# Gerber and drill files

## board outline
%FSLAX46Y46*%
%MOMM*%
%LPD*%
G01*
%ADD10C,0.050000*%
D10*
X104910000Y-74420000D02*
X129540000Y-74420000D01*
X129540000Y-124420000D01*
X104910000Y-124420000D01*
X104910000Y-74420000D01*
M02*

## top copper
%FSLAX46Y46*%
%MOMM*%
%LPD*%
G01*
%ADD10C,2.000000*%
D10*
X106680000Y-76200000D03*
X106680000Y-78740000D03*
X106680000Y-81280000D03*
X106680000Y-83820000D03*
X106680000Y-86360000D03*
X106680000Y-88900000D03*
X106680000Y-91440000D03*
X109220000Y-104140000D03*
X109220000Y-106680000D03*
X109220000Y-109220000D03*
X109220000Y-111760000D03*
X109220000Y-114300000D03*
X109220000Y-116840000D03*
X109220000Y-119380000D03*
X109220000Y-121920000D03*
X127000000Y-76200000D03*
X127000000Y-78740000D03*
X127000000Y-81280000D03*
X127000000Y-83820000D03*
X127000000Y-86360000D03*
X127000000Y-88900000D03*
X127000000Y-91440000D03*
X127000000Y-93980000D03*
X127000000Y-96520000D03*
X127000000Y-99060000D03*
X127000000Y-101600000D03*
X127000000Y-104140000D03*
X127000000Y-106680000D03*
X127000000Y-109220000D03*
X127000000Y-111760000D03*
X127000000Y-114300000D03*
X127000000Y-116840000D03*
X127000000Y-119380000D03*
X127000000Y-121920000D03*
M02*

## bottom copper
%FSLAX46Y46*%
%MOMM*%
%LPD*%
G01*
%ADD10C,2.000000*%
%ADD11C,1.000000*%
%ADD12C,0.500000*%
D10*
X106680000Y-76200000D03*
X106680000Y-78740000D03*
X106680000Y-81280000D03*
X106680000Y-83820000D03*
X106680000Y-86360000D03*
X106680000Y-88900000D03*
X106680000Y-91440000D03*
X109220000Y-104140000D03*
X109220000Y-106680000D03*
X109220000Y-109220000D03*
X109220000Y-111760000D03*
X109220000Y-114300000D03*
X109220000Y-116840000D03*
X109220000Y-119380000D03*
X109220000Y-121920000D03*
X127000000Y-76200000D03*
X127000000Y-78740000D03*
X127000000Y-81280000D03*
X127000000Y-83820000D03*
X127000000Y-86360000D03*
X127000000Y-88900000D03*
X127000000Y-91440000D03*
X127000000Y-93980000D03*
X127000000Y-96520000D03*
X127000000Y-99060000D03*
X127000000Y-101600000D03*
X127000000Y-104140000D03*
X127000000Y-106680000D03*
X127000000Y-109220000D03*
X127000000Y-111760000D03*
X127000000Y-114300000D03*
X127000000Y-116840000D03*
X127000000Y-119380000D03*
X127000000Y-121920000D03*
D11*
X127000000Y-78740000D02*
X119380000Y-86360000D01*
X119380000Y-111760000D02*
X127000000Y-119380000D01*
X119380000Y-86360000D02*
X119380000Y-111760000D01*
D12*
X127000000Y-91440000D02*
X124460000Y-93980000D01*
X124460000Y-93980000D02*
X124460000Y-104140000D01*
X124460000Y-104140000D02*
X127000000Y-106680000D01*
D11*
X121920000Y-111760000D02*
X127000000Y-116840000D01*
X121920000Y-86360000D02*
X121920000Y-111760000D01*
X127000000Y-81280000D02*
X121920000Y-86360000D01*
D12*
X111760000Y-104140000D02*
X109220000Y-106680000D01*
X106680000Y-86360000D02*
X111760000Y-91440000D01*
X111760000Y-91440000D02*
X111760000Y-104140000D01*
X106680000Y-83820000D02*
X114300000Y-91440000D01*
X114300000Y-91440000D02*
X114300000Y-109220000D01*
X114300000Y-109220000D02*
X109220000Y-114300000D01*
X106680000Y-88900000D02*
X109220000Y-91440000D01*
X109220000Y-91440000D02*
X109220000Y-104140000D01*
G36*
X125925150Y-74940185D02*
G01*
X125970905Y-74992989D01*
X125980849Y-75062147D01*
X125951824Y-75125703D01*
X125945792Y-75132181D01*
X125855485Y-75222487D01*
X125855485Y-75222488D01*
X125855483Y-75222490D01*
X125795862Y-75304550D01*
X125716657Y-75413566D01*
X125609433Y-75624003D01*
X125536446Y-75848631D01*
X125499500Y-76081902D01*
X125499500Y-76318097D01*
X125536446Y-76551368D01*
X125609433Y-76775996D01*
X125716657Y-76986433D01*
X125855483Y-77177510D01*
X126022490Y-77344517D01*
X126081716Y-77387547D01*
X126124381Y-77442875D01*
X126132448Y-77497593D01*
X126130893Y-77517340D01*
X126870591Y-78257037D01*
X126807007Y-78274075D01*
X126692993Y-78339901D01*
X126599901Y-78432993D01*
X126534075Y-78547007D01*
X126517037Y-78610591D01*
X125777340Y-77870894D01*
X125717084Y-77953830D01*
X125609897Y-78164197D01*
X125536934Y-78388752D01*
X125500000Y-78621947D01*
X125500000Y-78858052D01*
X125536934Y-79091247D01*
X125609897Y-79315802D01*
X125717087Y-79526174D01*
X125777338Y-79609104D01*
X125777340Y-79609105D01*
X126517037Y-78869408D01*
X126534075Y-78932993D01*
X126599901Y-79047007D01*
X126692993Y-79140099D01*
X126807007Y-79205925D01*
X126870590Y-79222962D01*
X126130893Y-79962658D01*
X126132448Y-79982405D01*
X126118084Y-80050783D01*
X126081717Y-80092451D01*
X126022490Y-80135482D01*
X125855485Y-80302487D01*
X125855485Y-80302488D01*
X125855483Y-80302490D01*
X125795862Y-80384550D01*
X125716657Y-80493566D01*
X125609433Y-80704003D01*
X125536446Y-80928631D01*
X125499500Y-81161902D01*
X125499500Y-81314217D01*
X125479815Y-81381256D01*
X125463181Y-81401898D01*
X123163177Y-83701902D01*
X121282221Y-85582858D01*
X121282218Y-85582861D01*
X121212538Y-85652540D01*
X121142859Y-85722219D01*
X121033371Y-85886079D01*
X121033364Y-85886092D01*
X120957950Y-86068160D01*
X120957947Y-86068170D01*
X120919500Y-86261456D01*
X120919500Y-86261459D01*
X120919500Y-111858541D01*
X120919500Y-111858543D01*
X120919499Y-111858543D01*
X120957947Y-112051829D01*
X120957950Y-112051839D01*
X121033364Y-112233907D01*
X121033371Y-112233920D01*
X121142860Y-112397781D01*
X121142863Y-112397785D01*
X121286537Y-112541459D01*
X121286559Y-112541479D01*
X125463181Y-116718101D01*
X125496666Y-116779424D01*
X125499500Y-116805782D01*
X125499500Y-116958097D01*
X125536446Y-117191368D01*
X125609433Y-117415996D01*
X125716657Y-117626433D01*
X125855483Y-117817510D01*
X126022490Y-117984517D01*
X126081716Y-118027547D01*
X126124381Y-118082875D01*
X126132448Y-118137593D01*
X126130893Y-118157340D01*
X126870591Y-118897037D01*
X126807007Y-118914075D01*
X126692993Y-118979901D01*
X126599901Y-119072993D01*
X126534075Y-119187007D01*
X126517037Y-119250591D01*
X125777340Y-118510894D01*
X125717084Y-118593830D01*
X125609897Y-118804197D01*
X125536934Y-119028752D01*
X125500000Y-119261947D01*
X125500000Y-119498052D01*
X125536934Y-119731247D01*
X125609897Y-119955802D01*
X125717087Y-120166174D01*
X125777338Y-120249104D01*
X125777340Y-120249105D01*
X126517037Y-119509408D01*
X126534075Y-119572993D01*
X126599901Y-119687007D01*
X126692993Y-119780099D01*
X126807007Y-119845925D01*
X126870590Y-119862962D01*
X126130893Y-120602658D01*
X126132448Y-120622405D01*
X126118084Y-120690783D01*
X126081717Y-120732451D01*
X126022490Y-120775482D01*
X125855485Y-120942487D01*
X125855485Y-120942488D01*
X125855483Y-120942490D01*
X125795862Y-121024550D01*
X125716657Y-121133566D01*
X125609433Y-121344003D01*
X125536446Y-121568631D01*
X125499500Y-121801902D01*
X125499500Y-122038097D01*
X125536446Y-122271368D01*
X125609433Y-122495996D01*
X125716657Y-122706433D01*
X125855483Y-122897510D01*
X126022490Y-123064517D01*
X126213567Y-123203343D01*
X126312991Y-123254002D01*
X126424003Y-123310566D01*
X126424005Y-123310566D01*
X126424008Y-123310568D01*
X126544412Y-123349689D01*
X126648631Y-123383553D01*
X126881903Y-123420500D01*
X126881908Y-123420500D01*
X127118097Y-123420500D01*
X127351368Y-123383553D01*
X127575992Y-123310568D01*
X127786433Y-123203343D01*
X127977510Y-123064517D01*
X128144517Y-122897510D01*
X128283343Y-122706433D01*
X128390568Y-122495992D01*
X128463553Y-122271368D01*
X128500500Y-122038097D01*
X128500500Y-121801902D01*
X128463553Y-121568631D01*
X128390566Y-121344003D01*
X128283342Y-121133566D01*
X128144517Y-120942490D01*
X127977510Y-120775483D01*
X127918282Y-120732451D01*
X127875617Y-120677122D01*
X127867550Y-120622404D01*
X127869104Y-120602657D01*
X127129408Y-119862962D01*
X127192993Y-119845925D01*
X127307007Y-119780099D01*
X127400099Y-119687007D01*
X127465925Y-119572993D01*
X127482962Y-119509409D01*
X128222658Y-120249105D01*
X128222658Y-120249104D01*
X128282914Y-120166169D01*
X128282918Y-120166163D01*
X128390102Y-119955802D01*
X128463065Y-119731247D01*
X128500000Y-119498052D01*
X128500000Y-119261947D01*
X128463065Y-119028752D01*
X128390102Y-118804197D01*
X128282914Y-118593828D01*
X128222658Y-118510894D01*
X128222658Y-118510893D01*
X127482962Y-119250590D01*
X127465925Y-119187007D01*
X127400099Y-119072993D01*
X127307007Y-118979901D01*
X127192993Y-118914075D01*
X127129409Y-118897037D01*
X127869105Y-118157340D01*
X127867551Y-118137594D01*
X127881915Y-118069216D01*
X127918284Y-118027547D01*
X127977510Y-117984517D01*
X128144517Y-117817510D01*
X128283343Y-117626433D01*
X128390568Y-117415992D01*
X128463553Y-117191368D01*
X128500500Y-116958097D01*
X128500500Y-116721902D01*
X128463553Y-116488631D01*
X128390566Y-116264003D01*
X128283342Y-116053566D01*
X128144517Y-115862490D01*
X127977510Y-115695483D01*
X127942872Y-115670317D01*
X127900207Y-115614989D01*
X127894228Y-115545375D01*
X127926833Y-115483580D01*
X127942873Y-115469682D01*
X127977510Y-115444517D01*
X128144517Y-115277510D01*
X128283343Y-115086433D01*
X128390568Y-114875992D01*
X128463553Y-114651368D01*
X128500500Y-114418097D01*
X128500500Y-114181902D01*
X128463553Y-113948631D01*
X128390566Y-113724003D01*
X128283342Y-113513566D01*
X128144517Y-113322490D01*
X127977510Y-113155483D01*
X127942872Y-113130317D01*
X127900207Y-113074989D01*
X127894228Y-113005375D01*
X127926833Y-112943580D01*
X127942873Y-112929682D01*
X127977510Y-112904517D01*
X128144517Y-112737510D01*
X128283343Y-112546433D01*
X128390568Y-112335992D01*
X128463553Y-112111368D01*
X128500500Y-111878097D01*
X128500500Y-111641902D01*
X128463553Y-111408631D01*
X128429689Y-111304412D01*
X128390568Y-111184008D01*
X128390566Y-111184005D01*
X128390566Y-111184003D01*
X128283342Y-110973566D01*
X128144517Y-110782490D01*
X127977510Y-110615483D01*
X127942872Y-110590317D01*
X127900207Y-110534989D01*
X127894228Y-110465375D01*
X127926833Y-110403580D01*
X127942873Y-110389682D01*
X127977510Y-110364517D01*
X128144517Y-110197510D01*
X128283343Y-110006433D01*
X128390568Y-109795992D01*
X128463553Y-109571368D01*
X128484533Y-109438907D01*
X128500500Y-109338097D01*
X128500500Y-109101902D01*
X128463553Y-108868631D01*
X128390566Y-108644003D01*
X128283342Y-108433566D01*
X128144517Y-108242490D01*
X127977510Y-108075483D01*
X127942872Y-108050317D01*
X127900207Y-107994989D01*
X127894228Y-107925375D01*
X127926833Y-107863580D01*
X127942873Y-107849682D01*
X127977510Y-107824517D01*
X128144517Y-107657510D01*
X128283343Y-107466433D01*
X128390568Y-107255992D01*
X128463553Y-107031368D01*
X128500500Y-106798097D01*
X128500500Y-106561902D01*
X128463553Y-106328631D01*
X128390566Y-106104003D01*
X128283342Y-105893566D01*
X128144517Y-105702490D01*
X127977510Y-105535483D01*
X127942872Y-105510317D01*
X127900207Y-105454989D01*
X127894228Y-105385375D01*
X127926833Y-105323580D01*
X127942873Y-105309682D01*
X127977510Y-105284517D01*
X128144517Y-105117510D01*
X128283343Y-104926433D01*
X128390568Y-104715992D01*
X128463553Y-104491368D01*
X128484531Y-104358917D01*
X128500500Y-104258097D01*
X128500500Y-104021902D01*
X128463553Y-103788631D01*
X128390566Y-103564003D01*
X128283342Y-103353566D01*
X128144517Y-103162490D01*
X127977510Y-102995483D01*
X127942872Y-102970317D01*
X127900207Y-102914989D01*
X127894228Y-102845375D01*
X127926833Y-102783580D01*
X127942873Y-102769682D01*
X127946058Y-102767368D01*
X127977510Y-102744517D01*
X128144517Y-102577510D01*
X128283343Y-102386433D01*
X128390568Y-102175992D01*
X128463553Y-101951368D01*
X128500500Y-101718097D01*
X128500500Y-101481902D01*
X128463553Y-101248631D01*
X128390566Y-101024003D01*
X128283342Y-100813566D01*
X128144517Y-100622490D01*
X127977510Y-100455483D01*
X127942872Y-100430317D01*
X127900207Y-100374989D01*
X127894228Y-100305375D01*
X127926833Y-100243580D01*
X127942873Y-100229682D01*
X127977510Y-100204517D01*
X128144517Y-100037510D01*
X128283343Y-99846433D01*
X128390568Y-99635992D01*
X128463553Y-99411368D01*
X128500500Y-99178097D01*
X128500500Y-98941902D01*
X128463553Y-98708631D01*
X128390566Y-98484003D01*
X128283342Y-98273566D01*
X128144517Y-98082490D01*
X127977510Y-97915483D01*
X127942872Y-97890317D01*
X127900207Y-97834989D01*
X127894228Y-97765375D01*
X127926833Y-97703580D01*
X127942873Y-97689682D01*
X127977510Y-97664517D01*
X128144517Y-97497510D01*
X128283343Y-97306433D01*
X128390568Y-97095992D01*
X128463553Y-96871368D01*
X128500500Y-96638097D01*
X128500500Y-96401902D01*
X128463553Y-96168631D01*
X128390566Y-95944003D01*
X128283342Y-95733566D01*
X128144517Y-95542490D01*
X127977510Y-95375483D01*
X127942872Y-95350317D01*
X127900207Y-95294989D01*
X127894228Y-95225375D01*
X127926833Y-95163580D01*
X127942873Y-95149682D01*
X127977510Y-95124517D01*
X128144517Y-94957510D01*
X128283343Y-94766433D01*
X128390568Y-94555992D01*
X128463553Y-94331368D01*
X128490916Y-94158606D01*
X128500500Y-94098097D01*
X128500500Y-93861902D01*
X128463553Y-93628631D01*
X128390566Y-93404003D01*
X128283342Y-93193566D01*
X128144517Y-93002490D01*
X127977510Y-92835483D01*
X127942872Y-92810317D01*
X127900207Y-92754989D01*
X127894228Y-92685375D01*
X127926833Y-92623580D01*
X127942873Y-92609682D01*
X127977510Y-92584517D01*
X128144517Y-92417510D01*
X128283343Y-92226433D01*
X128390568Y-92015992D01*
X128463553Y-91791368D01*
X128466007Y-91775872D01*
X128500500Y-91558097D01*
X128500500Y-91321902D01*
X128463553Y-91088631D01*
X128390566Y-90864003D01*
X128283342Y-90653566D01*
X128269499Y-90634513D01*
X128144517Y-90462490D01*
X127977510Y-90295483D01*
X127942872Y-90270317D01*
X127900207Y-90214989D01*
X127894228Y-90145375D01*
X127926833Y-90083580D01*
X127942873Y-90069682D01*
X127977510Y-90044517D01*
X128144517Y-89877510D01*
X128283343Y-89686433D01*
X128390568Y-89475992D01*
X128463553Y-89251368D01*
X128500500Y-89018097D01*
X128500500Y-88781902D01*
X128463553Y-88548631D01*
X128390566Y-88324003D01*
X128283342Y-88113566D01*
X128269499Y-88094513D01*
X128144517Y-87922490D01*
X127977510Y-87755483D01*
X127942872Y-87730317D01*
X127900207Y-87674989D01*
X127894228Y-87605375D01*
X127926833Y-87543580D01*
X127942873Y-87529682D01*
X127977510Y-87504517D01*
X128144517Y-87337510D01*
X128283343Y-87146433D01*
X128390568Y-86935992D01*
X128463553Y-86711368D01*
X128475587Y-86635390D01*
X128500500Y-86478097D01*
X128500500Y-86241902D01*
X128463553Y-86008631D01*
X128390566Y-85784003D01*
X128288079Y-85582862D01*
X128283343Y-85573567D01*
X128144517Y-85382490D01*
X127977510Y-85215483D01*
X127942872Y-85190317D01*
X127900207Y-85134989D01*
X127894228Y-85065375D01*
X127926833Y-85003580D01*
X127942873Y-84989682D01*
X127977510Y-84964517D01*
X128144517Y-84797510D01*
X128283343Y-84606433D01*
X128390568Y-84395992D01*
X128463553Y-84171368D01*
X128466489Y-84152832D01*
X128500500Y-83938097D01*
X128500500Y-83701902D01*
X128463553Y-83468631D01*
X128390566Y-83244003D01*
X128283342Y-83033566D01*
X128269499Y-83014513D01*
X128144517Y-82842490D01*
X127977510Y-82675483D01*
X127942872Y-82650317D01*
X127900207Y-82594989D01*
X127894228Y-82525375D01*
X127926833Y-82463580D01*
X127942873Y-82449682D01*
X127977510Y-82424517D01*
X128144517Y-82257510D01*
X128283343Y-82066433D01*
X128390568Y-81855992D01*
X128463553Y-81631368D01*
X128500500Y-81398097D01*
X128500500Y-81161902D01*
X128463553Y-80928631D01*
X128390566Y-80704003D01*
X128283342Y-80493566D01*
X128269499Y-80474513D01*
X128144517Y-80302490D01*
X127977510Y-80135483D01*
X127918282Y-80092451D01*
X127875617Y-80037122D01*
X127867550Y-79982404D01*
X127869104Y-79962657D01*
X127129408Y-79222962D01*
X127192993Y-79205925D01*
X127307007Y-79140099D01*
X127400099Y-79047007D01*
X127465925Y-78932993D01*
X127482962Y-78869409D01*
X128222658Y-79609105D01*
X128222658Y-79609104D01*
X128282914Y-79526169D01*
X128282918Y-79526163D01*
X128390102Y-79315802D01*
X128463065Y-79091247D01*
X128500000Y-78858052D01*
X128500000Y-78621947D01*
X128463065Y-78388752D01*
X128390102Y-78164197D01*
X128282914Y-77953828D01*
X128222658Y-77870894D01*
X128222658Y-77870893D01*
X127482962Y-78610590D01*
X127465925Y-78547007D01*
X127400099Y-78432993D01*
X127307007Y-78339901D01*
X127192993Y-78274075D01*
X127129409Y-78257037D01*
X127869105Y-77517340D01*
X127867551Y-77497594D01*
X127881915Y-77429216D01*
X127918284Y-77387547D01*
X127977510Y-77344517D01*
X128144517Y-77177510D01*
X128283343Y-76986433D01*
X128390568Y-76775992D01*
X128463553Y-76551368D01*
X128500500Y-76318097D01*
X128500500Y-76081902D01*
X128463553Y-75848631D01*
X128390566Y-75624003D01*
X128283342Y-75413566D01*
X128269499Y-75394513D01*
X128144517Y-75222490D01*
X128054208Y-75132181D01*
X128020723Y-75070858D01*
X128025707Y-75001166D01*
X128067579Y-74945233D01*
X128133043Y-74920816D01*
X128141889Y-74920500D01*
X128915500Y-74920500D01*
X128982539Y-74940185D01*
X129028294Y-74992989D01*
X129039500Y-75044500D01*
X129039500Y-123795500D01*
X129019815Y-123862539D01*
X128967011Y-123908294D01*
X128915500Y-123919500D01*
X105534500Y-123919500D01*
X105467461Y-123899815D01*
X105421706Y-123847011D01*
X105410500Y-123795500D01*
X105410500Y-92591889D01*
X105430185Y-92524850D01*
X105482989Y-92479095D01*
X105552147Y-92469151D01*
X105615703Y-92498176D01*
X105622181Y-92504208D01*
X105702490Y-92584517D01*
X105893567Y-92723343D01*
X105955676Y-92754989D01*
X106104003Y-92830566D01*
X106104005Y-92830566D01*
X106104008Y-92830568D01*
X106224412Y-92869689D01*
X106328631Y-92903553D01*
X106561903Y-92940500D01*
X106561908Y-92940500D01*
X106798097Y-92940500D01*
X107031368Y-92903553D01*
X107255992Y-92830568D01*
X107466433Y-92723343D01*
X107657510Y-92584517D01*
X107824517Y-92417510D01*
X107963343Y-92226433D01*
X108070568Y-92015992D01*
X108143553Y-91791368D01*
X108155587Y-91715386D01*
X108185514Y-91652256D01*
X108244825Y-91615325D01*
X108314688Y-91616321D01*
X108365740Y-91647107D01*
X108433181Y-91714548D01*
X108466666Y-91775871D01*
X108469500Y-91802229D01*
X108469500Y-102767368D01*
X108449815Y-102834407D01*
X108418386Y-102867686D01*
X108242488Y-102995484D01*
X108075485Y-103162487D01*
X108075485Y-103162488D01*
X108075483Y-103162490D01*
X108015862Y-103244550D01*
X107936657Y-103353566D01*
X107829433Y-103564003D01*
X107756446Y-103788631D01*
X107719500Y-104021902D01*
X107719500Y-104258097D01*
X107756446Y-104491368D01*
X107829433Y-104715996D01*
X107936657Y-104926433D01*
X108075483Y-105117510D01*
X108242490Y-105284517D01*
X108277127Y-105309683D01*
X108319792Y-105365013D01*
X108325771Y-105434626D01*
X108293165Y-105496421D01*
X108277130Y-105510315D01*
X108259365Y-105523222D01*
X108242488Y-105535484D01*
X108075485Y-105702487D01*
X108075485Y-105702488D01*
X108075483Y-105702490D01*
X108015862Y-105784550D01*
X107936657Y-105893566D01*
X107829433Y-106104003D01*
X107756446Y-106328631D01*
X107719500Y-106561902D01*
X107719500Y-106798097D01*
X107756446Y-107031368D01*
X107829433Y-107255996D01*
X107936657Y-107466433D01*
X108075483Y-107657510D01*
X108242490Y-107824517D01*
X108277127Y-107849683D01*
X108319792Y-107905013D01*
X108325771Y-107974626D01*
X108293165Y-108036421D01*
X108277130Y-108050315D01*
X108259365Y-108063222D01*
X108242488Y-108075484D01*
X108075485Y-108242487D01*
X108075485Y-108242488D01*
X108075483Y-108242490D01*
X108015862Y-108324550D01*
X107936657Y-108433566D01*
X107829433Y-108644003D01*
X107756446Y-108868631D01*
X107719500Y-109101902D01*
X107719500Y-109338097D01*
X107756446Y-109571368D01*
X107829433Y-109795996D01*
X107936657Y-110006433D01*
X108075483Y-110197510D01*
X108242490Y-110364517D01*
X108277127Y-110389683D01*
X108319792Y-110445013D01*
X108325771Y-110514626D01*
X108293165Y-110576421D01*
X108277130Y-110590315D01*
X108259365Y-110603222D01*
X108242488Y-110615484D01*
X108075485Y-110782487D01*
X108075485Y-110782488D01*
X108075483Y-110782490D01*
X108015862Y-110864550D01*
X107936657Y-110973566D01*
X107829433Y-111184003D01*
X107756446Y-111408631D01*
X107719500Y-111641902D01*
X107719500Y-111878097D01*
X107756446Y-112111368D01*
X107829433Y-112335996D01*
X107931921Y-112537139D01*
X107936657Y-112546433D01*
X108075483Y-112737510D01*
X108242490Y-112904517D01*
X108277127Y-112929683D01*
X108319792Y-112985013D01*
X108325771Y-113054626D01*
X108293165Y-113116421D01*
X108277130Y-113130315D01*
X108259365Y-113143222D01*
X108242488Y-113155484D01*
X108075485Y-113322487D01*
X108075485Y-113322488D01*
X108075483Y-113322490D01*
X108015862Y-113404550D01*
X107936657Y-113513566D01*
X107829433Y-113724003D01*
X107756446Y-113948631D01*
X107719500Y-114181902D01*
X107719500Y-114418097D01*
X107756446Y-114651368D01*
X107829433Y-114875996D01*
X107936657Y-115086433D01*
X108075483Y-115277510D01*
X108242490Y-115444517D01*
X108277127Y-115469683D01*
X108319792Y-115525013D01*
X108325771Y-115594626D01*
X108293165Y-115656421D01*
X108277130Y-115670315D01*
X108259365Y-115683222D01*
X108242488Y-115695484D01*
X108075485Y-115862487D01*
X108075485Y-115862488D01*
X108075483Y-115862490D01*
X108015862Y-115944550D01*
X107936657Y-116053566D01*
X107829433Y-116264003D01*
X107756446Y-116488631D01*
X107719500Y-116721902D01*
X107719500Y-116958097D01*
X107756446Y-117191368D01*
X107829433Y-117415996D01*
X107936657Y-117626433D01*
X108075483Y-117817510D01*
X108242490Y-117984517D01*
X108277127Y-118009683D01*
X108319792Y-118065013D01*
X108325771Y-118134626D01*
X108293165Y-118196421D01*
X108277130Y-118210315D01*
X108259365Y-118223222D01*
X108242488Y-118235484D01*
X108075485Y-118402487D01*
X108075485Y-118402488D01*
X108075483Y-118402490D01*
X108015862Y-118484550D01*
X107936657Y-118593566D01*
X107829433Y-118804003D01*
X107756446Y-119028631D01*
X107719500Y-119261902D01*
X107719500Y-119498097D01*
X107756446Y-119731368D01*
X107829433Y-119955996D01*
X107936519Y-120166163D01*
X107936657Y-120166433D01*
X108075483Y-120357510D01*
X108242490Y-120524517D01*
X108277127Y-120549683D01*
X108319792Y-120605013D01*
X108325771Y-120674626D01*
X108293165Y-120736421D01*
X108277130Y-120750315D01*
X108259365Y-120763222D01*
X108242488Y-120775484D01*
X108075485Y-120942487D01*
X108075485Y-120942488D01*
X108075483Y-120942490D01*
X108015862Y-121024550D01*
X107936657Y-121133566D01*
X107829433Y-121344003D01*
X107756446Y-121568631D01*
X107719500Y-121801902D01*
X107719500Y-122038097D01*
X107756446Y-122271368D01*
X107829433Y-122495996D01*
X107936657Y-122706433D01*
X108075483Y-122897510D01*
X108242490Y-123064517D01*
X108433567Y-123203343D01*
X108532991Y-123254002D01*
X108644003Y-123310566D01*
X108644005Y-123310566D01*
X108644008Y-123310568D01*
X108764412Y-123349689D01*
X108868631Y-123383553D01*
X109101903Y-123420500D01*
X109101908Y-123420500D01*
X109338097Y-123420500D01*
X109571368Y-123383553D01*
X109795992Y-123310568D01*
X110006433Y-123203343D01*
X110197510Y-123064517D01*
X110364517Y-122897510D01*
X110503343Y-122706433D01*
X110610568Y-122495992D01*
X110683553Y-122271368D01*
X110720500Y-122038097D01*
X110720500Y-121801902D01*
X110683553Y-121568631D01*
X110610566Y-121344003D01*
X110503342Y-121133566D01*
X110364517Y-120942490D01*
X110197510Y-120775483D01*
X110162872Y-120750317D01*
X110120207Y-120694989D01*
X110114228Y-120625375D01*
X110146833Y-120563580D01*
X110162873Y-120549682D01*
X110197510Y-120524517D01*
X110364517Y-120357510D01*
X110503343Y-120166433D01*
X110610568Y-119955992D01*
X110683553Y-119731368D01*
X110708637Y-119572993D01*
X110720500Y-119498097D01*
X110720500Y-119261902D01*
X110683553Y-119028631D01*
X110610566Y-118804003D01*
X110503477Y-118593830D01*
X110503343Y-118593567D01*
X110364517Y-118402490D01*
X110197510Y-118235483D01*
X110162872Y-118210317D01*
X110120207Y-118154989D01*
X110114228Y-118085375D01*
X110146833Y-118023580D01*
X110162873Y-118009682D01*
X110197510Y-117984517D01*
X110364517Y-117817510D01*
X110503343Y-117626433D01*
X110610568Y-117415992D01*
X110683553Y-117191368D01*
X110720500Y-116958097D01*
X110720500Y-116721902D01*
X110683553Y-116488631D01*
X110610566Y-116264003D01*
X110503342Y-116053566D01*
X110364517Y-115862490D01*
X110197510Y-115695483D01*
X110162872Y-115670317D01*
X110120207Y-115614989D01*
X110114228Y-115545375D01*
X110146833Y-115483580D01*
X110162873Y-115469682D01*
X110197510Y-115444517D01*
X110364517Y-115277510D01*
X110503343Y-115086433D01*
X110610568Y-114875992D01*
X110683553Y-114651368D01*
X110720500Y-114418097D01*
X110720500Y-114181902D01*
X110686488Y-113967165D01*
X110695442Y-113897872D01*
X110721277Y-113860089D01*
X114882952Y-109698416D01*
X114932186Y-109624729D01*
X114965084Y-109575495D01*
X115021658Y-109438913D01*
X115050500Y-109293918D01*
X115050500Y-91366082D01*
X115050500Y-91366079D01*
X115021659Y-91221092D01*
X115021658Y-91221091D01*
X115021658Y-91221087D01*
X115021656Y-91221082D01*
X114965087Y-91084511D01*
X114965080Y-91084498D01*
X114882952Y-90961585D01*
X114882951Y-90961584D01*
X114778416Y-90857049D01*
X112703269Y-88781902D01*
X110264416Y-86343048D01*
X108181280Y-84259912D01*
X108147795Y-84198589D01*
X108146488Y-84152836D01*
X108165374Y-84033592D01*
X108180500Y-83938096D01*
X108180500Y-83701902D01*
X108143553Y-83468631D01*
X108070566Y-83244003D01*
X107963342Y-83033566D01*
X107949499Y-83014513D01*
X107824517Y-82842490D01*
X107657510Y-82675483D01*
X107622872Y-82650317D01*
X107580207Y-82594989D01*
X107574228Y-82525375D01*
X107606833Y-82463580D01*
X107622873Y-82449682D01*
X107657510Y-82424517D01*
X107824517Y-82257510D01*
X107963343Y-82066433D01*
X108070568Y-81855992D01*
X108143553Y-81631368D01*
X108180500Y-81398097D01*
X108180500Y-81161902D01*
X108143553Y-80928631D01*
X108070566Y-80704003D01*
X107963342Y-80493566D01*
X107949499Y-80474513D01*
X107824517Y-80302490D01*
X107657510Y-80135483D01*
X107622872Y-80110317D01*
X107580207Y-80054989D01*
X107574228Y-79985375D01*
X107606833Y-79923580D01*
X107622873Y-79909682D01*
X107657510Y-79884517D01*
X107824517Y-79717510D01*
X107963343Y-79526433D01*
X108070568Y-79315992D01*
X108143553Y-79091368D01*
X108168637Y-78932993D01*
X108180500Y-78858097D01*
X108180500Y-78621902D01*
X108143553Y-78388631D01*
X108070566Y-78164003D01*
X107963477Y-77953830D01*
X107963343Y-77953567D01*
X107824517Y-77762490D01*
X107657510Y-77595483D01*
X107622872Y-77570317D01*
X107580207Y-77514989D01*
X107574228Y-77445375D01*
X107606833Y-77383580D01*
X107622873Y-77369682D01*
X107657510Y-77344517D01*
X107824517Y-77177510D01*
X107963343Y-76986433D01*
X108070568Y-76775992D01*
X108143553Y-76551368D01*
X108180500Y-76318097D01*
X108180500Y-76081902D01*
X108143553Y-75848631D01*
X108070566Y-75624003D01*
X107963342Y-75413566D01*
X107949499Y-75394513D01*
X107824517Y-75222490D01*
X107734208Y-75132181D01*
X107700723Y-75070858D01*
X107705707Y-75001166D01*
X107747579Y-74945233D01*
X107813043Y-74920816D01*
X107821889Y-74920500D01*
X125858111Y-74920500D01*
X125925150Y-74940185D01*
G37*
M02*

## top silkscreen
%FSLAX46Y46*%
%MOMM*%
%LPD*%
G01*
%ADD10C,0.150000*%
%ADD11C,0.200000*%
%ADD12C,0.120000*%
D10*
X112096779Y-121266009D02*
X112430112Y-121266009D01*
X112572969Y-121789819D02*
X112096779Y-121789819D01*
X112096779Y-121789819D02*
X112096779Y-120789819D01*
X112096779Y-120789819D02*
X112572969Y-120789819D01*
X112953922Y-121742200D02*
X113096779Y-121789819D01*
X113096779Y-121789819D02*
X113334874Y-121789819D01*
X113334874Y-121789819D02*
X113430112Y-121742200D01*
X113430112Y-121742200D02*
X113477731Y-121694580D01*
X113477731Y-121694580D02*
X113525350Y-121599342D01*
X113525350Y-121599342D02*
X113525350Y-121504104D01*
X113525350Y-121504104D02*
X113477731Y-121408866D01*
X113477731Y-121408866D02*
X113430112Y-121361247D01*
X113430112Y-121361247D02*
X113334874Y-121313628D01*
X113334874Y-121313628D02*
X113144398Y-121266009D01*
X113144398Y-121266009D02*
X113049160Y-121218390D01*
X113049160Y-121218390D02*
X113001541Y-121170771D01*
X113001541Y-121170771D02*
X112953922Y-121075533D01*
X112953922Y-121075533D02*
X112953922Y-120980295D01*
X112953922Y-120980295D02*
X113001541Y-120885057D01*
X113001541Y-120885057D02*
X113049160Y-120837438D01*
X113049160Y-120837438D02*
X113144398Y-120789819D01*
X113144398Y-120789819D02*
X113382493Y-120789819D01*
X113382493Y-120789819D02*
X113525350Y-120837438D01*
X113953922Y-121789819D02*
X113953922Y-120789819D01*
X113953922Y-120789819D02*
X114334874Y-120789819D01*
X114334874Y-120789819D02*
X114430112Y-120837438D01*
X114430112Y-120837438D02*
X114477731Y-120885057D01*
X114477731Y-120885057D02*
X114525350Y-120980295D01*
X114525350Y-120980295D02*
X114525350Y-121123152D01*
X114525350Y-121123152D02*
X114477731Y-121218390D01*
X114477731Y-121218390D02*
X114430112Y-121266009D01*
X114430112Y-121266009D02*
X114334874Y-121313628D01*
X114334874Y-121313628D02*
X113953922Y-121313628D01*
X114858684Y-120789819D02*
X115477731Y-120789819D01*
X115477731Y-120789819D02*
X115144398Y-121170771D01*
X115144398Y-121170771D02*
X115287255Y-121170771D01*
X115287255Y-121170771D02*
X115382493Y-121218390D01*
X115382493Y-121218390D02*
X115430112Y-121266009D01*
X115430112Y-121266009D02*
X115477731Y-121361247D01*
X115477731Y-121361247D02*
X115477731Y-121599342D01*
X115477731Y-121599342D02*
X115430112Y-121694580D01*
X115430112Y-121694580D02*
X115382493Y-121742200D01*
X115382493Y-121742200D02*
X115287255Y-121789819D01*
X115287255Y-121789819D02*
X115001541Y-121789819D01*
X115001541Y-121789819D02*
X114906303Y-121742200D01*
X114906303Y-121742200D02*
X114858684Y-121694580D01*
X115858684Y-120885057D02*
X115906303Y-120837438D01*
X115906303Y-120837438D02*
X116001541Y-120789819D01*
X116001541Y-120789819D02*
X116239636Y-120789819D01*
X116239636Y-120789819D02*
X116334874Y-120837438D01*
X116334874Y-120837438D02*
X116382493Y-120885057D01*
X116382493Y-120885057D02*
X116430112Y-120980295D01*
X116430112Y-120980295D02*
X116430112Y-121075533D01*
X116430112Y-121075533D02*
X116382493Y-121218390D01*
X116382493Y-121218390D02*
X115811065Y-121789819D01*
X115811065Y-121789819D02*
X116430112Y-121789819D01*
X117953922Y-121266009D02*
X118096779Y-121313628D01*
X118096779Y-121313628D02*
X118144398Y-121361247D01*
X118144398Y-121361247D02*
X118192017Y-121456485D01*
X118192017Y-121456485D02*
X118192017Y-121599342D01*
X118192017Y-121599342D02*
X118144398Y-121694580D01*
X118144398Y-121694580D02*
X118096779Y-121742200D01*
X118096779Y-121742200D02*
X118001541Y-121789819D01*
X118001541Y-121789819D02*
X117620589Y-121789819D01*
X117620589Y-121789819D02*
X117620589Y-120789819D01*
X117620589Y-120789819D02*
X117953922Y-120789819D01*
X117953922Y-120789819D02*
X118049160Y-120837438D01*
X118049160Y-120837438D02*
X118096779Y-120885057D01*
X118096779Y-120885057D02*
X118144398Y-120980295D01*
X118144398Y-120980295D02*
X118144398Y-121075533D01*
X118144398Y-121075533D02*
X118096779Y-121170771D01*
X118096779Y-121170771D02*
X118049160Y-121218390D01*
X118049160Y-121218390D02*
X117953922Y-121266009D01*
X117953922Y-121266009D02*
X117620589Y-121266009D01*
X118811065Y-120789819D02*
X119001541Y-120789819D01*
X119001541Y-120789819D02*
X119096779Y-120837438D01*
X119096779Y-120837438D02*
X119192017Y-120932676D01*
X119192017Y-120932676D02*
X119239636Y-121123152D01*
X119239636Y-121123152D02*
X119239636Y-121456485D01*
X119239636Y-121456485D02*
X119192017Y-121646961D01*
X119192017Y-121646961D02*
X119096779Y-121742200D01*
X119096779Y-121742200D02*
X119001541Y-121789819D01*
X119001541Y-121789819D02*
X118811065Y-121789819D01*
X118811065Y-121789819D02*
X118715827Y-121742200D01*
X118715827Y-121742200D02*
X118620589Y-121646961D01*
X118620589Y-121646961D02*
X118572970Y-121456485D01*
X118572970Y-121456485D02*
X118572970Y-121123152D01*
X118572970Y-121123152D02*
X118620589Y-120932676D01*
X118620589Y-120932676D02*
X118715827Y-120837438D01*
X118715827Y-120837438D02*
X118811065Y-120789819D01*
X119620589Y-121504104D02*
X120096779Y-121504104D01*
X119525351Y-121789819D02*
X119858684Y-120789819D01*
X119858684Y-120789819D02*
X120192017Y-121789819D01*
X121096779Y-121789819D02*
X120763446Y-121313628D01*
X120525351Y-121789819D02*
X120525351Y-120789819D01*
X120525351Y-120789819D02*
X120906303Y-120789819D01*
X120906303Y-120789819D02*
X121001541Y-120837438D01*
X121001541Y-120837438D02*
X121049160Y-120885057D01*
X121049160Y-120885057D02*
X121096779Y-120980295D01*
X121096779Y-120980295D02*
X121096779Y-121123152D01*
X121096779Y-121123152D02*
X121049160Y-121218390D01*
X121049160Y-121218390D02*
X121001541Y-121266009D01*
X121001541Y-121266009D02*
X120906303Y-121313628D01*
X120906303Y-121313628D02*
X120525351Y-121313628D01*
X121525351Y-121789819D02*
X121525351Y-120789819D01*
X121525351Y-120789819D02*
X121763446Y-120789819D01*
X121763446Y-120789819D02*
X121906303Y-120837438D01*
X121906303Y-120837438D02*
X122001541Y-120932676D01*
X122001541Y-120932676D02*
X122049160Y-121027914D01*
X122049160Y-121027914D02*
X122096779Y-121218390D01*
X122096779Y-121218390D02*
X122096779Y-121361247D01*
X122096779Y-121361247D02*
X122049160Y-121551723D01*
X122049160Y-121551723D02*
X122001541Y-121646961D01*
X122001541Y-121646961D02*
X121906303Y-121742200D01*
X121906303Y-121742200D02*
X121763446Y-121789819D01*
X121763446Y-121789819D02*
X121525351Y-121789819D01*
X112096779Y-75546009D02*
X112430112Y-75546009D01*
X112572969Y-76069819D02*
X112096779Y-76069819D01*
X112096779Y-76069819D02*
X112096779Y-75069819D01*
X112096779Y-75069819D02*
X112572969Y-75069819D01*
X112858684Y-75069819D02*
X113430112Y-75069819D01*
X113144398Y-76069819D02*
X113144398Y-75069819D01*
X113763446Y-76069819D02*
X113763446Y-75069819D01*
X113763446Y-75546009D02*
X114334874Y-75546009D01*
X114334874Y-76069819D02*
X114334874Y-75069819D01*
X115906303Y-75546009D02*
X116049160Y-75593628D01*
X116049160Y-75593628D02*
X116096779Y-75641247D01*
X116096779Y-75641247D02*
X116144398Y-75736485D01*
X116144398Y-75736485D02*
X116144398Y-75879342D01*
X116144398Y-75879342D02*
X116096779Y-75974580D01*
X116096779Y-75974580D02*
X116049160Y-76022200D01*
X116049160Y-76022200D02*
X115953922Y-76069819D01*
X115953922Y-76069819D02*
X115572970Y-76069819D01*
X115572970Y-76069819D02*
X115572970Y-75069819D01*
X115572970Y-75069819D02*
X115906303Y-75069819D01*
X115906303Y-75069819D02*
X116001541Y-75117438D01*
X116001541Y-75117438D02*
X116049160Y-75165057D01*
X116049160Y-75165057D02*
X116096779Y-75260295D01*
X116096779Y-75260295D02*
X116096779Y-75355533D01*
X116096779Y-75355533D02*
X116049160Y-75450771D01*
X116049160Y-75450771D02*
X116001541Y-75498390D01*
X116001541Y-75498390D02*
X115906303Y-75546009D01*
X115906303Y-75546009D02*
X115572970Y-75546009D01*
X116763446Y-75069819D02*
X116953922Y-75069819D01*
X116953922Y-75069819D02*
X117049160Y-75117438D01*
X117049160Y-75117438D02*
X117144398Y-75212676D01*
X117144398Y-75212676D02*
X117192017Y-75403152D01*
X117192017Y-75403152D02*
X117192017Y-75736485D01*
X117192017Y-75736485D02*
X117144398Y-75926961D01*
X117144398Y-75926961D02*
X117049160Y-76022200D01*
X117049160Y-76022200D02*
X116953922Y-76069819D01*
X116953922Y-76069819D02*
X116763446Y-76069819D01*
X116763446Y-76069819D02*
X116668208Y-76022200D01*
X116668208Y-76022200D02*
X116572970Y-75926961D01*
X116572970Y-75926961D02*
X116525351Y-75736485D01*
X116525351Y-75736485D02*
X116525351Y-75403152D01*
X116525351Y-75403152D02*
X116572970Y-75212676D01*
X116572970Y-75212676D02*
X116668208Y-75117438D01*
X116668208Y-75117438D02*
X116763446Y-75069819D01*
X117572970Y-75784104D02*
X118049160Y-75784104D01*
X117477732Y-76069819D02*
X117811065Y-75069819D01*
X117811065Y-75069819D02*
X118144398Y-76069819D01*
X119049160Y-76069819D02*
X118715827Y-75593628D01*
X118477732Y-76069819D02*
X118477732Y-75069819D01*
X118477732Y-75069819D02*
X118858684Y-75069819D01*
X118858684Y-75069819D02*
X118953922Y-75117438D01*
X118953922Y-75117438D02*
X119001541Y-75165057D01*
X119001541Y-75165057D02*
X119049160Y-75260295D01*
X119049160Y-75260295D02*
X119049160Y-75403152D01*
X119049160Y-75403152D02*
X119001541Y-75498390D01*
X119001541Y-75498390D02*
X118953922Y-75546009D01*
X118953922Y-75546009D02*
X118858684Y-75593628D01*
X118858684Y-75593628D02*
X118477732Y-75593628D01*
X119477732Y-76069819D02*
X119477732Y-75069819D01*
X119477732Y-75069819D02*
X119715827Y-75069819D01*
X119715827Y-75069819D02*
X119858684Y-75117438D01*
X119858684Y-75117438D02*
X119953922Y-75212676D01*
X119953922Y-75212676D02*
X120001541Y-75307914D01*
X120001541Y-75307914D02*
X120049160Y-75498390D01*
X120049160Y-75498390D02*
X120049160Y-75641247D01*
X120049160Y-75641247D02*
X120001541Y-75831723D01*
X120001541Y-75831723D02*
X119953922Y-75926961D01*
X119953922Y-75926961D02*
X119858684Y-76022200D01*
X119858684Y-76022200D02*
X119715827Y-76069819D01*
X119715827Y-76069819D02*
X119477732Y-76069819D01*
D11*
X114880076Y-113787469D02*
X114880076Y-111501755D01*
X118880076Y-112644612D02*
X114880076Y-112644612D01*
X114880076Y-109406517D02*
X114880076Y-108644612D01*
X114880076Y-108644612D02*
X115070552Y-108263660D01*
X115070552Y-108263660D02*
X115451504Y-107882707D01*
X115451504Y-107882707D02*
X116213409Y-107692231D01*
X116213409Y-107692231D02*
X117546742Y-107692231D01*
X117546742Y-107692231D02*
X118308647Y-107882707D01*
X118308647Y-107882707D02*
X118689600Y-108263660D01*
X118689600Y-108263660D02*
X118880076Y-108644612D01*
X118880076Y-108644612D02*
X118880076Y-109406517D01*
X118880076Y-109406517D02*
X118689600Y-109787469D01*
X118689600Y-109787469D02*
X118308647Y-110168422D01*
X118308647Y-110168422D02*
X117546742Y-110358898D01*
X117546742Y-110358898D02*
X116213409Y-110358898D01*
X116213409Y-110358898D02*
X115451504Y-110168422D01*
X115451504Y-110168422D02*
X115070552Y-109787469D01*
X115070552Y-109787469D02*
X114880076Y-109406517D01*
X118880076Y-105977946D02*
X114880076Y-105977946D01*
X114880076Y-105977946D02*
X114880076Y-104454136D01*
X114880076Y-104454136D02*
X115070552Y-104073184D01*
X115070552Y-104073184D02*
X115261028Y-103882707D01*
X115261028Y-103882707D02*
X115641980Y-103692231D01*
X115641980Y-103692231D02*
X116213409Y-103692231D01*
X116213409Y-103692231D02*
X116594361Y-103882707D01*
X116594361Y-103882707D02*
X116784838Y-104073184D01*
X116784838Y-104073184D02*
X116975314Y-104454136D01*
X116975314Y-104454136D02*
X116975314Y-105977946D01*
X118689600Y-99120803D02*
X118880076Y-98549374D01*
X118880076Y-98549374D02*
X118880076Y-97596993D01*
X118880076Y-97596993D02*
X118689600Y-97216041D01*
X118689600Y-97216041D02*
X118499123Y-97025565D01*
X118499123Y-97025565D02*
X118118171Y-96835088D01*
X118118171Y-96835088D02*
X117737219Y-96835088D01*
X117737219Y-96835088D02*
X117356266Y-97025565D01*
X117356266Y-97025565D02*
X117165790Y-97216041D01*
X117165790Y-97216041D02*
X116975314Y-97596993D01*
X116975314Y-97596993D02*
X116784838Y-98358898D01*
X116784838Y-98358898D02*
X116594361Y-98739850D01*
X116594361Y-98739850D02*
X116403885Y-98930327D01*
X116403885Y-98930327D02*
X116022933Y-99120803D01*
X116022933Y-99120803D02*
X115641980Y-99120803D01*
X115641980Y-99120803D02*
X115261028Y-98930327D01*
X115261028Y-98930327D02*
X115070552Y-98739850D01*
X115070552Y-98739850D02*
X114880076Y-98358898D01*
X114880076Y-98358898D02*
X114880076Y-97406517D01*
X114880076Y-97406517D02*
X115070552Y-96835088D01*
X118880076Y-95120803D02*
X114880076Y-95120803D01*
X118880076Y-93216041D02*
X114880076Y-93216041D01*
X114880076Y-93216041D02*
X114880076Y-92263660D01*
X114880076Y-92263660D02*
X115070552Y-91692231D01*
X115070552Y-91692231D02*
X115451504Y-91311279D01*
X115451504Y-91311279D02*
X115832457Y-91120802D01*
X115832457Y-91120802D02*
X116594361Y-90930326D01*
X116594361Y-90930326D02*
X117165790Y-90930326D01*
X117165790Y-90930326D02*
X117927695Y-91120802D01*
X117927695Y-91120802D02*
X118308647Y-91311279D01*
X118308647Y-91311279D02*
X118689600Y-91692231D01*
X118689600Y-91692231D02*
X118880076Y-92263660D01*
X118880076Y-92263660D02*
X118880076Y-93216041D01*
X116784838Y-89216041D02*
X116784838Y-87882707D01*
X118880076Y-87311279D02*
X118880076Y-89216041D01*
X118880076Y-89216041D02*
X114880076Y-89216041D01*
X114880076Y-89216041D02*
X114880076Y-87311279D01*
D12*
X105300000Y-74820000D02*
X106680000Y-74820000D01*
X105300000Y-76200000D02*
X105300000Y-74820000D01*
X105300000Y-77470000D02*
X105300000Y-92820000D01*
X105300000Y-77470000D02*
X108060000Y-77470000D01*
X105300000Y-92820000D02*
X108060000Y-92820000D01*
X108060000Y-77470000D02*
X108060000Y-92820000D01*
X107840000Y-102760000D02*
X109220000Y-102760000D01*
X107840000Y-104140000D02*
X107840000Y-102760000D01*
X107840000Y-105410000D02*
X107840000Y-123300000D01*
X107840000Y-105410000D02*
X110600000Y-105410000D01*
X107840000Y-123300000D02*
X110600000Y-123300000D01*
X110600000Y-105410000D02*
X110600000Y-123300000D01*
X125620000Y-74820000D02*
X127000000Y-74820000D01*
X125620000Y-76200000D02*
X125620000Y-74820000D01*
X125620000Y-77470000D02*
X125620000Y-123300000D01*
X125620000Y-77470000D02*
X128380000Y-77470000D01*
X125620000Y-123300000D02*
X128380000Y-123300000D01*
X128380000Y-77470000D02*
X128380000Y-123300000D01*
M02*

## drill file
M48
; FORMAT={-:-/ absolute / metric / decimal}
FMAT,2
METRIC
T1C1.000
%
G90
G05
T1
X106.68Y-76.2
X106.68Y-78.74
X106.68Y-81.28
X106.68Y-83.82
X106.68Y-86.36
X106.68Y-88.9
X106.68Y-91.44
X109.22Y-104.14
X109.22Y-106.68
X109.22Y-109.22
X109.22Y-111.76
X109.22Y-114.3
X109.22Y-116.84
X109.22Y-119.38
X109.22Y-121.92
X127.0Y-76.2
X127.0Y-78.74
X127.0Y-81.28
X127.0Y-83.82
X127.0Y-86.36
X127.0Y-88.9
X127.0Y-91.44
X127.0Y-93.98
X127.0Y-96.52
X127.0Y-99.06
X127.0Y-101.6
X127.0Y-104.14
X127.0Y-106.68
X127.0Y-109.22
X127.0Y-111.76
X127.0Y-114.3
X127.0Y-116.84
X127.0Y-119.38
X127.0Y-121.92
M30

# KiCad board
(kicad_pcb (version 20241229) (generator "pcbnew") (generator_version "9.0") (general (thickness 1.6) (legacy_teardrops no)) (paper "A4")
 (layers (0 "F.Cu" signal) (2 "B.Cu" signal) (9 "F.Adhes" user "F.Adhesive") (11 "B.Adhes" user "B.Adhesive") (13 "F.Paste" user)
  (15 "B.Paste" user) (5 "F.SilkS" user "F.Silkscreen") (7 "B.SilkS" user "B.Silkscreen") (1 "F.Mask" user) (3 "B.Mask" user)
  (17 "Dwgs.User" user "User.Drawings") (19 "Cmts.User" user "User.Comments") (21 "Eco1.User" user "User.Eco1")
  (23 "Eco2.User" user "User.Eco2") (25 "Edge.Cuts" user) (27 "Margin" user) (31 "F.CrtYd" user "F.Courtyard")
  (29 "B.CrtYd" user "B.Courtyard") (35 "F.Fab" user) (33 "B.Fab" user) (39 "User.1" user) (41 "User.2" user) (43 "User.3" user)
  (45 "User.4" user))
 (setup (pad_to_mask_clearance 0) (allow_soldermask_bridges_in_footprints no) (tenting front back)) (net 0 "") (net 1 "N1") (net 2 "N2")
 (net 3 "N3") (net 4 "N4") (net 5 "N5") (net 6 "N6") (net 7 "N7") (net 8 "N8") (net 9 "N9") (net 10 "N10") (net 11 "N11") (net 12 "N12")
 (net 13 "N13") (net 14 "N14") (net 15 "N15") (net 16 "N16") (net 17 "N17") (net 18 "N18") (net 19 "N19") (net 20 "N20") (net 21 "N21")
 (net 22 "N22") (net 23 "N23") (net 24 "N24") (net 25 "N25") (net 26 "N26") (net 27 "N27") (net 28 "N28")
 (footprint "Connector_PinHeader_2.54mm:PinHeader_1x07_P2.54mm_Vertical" (layer "F.Cu") (at 106.68 76.2)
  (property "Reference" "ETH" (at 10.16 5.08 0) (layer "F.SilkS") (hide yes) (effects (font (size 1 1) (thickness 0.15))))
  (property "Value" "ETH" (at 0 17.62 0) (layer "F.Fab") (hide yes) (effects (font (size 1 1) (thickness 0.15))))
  (fp_line (start -1.38 -1.38) (end 0 -1.38) (stroke (width 0.12) (type solid)) (layer "F.SilkS"))
  (fp_line (start -1.38 0) (end -1.38 -1.38) (stroke (width 0.12) (type solid)) (layer "F.SilkS"))
  (fp_line (start -1.38 1.27) (end -1.38 16.62) (stroke (width 0.12) (type solid)) (layer "F.SilkS"))
  (fp_line (start -1.38 1.27) (end 1.38 1.27) (stroke (width 0.12) (type solid)) (layer "F.SilkS"))
  (fp_line (start -1.38 16.62) (end 1.38 16.62) (stroke (width 0.12) (type solid)) (layer "F.SilkS"))
  (fp_line (start 1.38 1.27) (end 1.38 16.62) (stroke (width 0.12) (type solid)) (layer "F.SilkS"))
  (pad "1" thru_hole circle (at 0 0) (size 2 2) (drill 1) (layers "*.Cu" "*.Mask") (remove_unused_layers no) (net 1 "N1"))
  (pad "2" thru_hole circle (at 0 2.54) (size 2 2) (drill 1) (layers "*.Cu" "*.Mask") (remove_unused_layers no) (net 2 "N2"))
  (pad "3" thru_hole circle (at 0 5.08) (size 2 2) (drill 1) (layers "*.Cu" "*.Mask") (remove_unused_layers no) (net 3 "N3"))
  (pad "4" thru_hole circle (at 0 7.62) (size 2 2) (drill 1) (layers "*.Cu" "*.Mask") (remove_unused_layers no) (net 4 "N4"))
  (pad "5" thru_hole circle (at 0 10.16) (size 2 2) (drill 1) (layers "*.Cu" "*.Mask") (remove_unused_layers no) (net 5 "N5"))
  (pad "6" thru_hole circle (at 0 12.7) (size 2 2) (drill 1) (layers "*.Cu" "*.Mask") (remove_unused_layers no) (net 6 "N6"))
  (pad "7" thru_hole circle (at 0 15.24) (size 2 2) (drill 1) (layers "*.Cu" "*.Mask") (remove_unused_layers no) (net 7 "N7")))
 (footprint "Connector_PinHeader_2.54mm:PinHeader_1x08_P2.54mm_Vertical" (layer "F.Cu") (at 109.22 104.14)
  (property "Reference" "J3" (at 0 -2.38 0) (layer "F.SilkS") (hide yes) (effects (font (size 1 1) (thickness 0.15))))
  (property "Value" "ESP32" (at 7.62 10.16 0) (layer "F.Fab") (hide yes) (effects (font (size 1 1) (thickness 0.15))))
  (fp_line (start -1.38 -1.38) (end 0 -1.38) (stroke (width 0.12) (type solid)) (layer "F.SilkS"))
  (fp_line (start -1.38 0) (end -1.38 -1.38) (stroke (width 0.12) (type solid)) (layer "F.SilkS"))
  (fp_line (start -1.38 1.27) (end -1.38 19.16) (stroke (width 0.12) (type solid)) (layer "F.SilkS"))
  (fp_line (start -1.38 1.27) (end 1.38 1.27) (stroke (width 0.12) (type solid)) (layer "F.SilkS"))
  (fp_line (start -1.38 19.16) (end 1.38 19.16) (stroke (width 0.12) (type solid)) (layer "F.SilkS"))
  (fp_line (start 1.38 1.27) (end 1.38 19.16) (stroke (width 0.12) (type solid)) (layer "F.SilkS"))
  (pad "1" thru_hole circle (at 0 0) (size 2 2) (drill 1) (layers "*.Cu" "*.Mask") (remove_unused_layers no) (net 6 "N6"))
  (pad "2" thru_hole circle (at 0 2.54) (size 2 2) (drill 1) (layers "*.Cu" "*.Mask") (remove_unused_layers no) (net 5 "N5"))
  (pad "3" thru_hole circle (at 0 5.08) (size 2 2) (drill 1) (layers "*.Cu" "*.Mask") (remove_unused_layers no) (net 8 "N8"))
  (pad "4" thru_hole circle (at 0 7.62) (size 2 2) (drill 1) (layers "*.Cu" "*.Mask") (remove_unused_layers no) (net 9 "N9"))
  (pad "5" thru_hole circle (at 0 10.16) (size 2 2) (drill 1) (layers "*.Cu" "*.Mask") (remove_unused_layers no) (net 4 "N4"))
  (pad "6" thru_hole circle (at 0 12.7) (size 2 2) (drill 1) (layers "*.Cu" "*.Mask") (remove_unused_layers no) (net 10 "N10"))
  (pad "7" thru_hole circle (at 0 15.24) (size 2 2) (drill 1) (layers "*.Cu" "*.Mask") (remove_unused_layers no) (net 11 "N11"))
  (pad "8" thru_hole circle (at 0 17.78) (size 2 2) (drill 1) (layers "*.Cu" "*.Mask") (remove_unused_layers no) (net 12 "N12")))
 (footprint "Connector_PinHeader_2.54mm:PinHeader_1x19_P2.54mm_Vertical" (layer "F.Cu") (at 127 76.2)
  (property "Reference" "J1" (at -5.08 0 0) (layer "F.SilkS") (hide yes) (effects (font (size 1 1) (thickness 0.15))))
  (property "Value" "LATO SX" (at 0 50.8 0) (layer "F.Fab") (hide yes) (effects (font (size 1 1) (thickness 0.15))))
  (fp_line (start -1.38 -1.38) (end 0 -1.38) (stroke (width 0.12) (type solid)) (layer "F.SilkS"))
  (fp_line (start -1.38 0) (end -1.38 -1.38) (stroke (width 0.12) (type solid)) (layer "F.SilkS"))
  (fp_line (start -1.38 1.27) (end -1.38 47.1) (stroke (width 0.12) (type solid)) (layer "F.SilkS"))
  (fp_line (start -1.38 1.27) (end 1.38 1.27) (stroke (width 0.12) (type solid)) (layer "F.SilkS"))
  (fp_line (start -1.38 47.1) (end 1.38 47.1) (stroke (width 0.12) (type solid)) (layer "F.SilkS"))
  (fp_line (start 1.38 1.27) (end 1.38 47.1) (stroke (width 0.12) (type solid)) (layer "F.SilkS"))
  (pad "1" thru_hole circle (at 0 0) (size 2 2) (drill 1) (layers "*.Cu" "*.Mask") (remove_unused_layers no) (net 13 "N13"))
  (pad "2" thru_hole circle (at 0 2.54) (size 2 2) (drill 1) (layers "*.Cu" "*.Mask") (remove_unused_layers no) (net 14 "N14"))
  (pad "3" thru_hole circle (at 0 5.08) (size 2 2) (drill 1) (layers "*.Cu" "*.Mask") (remove_unused_layers no) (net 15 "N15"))
  (pad "4" thru_hole circle (at 0 7.62) (size 2 2) (drill 1) (layers "*.Cu" "*.Mask") (remove_unused_layers no) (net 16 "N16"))
  (pad "5" thru_hole circle (at 0 10.16) (size 2 2) (drill 1) (layers "*.Cu" "*.Mask") (remove_unused_layers no) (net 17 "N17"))
  (pad "6" thru_hole circle (at 0 12.7) (size 2 2) (drill 1) (layers "*.Cu" "*.Mask") (remove_unused_layers no) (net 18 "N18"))
  (pad "7" thru_hole circle (at 0 15.24) (size 2 2) (drill 1) (layers "*.Cu" "*.Mask") (remove_unused_layers no) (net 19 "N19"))
  (pad "8" thru_hole circle (at 0 17.78) (size 2 2) (drill 1) (layers "*.Cu" "*.Mask") (remove_unused_layers no) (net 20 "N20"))
  (pad "9" thru_hole circle (at 0 20.32) (size 2 2) (drill 1) (layers "*.Cu" "*.Mask") (remove_unused_layers no) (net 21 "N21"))
  (pad "10" thru_hole circle (at 0 22.86) (size 2 2) (drill 1) (layers "*.Cu" "*.Mask") (remove_unused_layers no) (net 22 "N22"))
  (pad "11" thru_hole circle (at 0 25.4) (size 2 2) (drill 1) (layers "*.Cu" "*.Mask") (remove_unused_layers no) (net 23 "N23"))
  (pad "12" thru_hole circle (at 0 27.94) (size 2 2) (drill 1) (layers "*.Cu" "*.Mask") (remove_unused_layers no) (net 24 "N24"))
  (pad "13" thru_hole circle (at 0 30.48) (size 2 2) (drill 1) (layers "*.Cu" "*.Mask") (remove_unused_layers no) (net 19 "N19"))
  (pad "14" thru_hole circle (at 0 33.02) (size 2 2) (drill 1) (layers "*.Cu" "*.Mask") (remove_unused_layers no) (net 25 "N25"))
  (pad "15" thru_hole circle (at 0 35.56) (size 2 2) (drill 1) (layers "*.Cu" "*.Mask") (remove_unused_layers no) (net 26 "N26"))
  (pad "16" thru_hole circle (at 0 38.1) (size 2 2) (drill 1) (layers "*.Cu" "*.Mask") (remove_unused_layers no) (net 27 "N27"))
  (pad "17" thru_hole circle (at 0 40.64) (size 2 2) (drill 1) (layers "*.Cu" "*.Mask") (remove_unused_layers no) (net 15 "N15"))
  (pad "18" thru_hole circle (at 0 43.18) (size 2 2) (drill 1) (layers "*.Cu" "*.Mask") (remove_unused_layers no) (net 14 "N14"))
  (pad "19" thru_hole circle (at 0 45.72) (size 2 2) (drill 1) (layers "*.Cu" "*.Mask") (remove_unused_layers no) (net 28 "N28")))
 (gr_rect (start 104.91 74.42) (end 129.54 124.42) (stroke (width 0.05) (type solid)) (fill no) (layer "Edge.Cuts"))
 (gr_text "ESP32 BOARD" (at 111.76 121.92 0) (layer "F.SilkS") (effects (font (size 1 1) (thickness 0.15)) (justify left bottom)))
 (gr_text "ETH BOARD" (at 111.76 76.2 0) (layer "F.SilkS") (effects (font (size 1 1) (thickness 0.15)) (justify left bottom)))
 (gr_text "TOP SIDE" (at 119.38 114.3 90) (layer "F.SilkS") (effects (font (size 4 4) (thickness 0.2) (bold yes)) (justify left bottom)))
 (segment (start 127 78.74) (end 119.38 86.36) (width 1) (layer "B.Cu") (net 14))
 (segment (start 119.38 111.76) (end 127 119.38) (width 1) (layer "B.Cu") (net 14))
 (segment (start 119.38 86.36) (end 119.38 111.76) (width 1) (layer "B.Cu") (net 14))
 (segment (start 127 91.44) (end 124.46 93.98) (width 0.5) (layer "B.Cu") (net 19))
 (segment (start 124.46 93.98) (end 124.46 104.14) (width 0.5) (layer "B.Cu") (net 19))
 (segment (start 124.46 104.14) (end 127 106.68) (width 0.5) (layer "B.Cu") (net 19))
 (segment (start 121.92 111.76) (end 127 116.84) (width 1) (layer "B.Cu") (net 15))
 (segment (start 121.92 86.36) (end 121.92 111.76) (width 1) (layer "B.Cu") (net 15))
 (segment (start 127 81.28) (end 121.92 86.36) (width 1) (layer "B.Cu") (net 15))
 (segment (start 111.76 104.14) (end 109.22 106.68) (width 0.5) (layer "B.Cu") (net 5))
 (segment (start 106.68 86.36) (end 111.76 91.44) (width 0.5) (layer "B.Cu") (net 5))
 (segment (start 111.76 91.44) (end 111.76 104.14) (width 0.5) (layer "B.Cu") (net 5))
 (segment (start 106.68 83.82) (end 114.3 91.44) (width 0.5) (layer "B.Cu") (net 4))
 (segment (start 114.3 91.44) (end 114.3 109.22) (width 0.5) (layer "B.Cu") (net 4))
 (segment (start 114.3 109.22) (end 109.22 114.3) (width 0.5) (layer "B.Cu") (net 4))
 (segment (start 106.68 88.9) (end 109.22 91.44) (width 0.5) (layer "B.Cu") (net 6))
 (segment (start 109.22 91.44) (end 109.22 104.14) (width 0.5) (layer "B.Cu") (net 6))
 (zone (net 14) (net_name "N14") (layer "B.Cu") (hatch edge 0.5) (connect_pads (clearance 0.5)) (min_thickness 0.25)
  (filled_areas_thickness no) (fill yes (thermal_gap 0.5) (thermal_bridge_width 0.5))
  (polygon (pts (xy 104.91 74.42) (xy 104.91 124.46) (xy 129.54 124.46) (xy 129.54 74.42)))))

